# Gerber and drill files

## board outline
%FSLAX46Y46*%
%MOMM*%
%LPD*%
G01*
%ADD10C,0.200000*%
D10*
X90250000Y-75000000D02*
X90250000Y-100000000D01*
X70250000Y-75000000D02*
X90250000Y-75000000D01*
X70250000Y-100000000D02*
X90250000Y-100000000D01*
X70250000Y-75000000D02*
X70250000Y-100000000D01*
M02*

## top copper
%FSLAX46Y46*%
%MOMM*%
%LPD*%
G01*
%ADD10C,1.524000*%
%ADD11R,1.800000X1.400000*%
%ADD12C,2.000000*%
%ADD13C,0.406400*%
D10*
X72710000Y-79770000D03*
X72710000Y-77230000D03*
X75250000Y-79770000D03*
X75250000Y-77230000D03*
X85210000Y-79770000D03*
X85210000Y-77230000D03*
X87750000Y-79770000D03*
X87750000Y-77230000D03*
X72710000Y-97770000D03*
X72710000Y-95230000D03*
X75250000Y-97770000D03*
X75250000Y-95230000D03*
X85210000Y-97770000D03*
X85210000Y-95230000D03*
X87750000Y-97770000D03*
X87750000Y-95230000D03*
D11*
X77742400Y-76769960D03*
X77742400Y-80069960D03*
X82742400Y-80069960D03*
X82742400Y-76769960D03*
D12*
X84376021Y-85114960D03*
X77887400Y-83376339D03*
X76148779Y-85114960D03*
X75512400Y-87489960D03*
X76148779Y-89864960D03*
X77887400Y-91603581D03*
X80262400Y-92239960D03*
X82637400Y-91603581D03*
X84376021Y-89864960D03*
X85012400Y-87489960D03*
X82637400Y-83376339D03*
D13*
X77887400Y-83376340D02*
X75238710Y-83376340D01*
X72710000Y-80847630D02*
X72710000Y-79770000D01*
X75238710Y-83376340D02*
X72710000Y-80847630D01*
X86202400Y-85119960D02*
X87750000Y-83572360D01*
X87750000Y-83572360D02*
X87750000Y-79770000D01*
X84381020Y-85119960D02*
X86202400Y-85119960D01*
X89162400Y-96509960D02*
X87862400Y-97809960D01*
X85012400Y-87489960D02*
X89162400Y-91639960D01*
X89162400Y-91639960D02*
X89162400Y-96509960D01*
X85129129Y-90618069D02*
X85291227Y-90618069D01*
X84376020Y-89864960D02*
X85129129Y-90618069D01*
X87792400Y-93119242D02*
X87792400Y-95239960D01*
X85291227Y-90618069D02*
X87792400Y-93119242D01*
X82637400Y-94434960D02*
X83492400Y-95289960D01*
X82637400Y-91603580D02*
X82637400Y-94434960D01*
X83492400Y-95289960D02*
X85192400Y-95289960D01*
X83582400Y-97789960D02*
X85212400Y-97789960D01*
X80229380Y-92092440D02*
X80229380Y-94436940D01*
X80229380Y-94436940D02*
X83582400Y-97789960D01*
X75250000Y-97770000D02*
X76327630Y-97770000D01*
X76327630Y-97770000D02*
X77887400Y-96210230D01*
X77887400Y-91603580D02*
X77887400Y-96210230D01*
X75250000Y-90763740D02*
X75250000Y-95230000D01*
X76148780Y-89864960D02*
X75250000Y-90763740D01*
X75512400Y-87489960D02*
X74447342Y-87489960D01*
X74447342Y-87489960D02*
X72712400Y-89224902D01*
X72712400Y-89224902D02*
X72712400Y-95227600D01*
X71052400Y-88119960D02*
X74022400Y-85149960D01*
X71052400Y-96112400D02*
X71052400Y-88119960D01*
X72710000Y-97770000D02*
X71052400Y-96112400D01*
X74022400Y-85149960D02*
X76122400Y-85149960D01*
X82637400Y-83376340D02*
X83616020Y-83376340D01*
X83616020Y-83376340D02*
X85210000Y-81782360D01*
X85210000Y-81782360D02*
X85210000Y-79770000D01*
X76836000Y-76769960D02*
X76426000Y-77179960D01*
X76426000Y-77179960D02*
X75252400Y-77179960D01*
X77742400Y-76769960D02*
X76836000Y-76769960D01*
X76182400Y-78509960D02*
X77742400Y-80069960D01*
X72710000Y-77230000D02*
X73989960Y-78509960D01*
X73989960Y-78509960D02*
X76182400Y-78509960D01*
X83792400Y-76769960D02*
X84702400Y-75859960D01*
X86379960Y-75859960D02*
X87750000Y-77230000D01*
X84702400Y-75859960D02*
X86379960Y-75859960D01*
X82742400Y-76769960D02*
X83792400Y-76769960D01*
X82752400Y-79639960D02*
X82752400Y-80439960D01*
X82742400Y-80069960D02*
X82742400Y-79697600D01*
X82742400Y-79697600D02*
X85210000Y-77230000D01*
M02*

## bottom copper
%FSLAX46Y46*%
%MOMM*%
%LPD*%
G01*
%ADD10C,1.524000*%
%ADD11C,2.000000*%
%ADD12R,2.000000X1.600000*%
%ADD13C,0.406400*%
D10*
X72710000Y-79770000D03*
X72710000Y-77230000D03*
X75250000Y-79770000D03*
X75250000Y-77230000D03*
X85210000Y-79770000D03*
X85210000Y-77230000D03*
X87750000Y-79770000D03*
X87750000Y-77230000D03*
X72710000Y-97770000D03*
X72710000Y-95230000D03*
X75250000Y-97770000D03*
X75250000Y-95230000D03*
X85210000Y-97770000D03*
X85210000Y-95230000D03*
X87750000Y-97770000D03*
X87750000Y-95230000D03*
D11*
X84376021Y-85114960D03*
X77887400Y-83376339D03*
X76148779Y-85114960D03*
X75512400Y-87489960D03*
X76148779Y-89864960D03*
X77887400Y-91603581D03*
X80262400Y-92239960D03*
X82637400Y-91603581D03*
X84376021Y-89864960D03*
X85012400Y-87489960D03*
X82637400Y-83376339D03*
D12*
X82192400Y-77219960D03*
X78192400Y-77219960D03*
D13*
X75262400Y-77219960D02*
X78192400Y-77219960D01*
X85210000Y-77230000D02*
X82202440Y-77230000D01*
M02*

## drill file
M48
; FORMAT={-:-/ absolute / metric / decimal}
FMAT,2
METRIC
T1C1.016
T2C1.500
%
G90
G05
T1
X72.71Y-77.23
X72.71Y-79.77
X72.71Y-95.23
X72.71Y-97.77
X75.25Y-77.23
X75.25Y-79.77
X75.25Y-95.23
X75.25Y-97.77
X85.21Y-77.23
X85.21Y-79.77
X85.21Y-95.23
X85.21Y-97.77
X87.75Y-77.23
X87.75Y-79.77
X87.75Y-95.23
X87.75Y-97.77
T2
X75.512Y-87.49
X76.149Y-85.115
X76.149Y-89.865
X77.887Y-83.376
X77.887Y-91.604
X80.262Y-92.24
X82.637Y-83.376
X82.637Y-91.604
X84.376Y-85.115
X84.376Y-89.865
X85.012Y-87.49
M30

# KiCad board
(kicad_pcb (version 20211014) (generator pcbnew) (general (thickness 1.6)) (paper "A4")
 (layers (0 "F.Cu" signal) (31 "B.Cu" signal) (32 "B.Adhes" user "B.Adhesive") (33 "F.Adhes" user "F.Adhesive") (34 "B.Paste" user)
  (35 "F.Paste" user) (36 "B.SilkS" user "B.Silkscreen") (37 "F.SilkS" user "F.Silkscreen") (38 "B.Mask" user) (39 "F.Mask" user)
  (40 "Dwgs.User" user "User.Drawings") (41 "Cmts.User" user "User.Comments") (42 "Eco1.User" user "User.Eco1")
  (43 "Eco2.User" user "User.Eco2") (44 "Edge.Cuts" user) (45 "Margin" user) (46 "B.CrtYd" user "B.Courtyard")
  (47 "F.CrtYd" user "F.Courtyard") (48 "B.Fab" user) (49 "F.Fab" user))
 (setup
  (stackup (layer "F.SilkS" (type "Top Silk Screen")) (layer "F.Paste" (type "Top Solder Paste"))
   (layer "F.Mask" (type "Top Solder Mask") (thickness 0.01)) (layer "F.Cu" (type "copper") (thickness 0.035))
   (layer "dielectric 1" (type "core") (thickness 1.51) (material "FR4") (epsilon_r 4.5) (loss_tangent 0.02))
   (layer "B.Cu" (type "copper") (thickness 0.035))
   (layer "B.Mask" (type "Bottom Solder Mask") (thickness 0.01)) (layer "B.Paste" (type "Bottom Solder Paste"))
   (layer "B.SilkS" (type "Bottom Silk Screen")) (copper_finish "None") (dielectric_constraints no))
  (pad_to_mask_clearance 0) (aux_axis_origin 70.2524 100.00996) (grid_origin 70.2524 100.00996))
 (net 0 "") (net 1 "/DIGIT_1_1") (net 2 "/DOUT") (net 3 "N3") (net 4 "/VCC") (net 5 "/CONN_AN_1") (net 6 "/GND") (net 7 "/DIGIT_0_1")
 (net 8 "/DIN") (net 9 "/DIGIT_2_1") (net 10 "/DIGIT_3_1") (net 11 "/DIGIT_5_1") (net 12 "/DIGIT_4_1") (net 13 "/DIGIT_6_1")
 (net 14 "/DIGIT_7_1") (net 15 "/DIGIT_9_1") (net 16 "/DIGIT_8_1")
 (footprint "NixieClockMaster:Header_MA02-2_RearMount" (layer "F.Cu") (at 75.25 78.5)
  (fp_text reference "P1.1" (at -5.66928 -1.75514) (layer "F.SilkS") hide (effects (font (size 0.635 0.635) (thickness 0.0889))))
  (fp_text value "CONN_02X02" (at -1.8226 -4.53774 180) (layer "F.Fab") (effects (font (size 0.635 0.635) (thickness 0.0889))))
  (pad "1" thru_hole circle (at -2.54 1.27) (size 1.524 1.524) (drill 1.016) (layers *.Cu *.Mask) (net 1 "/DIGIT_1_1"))
  (pad "2" thru_hole circle (at -2.54 -1.27) (size 1.524 1.524) (drill 1.016) (layers *.Cu *.Mask) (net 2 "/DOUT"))
  (pad "3" thru_hole circle (at 0 1.27) (size 1.524 1.524) (drill 1.016) (layers *.Cu *.Mask) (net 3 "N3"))
  (pad "4" thru_hole circle (at 0 -1.27) (size 1.524 1.524) (drill 1.016) (layers *.Cu *.Mask) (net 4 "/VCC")))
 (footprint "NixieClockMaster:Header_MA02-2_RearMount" (layer "F.Cu") (at 87.75 78.5)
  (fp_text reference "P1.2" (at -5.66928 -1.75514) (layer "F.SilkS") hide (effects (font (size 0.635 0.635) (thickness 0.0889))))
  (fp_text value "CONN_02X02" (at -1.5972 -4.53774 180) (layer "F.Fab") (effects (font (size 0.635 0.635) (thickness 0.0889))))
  (pad "1" thru_hole circle (at -2.54 1.27) (size 1.524 1.524) (drill 1.016) (layers *.Cu *.Mask) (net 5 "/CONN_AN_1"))
  (pad "2" thru_hole circle (at -2.54 -1.27) (size 1.524 1.524) (drill 1.016) (layers *.Cu *.Mask) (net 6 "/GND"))
  (pad "3" thru_hole circle (at 0 1.27) (size 1.524 1.524) (drill 1.016) (layers *.Cu *.Mask) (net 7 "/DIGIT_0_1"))
  (pad "4" thru_hole circle (at 0 -1.27) (size 1.524 1.524) (drill 1.016) (layers *.Cu *.Mask) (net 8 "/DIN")))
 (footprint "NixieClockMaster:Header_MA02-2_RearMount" (layer "F.Cu") (at 75.25 96.5)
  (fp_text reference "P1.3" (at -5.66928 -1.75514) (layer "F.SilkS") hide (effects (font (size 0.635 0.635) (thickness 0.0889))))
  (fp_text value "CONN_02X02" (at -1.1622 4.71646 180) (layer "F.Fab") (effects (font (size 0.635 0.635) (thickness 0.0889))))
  (pad "1" thru_hole circle (at -2.54 1.27) (size 1.524 1.524) (drill 1.016) (layers *.Cu *.Mask) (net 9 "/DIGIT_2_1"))
  (pad "2" thru_hole circle (at -2.54 -1.27) (size 1.524 1.524) (drill 1.016) (layers *.Cu *.Mask) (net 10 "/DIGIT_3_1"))
  (pad "3" thru_hole circle (at 0 1.27) (size 1.524 1.524) (drill 1.016) (layers *.Cu *.Mask) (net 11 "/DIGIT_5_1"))
  (pad "4" thru_hole circle (at 0 -1.27) (size 1.524 1.524) (drill 1.016) (layers *.Cu *.Mask) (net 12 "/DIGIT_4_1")))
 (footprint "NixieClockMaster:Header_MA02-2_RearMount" (layer "F.Cu") (at 87.75 96.5)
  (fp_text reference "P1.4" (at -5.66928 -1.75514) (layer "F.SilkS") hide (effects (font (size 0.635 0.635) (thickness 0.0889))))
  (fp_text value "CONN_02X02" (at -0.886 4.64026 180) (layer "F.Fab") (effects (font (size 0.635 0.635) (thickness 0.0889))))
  (pad "1" thru_hole circle (at -2.54 1.27) (size 1.524 1.524) (drill 1.016) (layers *.Cu *.Mask) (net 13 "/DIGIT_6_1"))
  (pad "2" thru_hole circle (at -2.54 -1.27) (size 1.524 1.524) (drill 1.016) (layers *.Cu *.Mask) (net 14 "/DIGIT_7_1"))
  (pad "3" thru_hole circle (at 0 1.27) (size 1.524 1.524) (drill 1.016) (layers *.Cu *.Mask) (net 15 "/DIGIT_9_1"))
  (pad "4" thru_hole circle (at 0 -1.27) (size 1.524 1.524) (drill 1.016) (layers *.Cu *.Mask) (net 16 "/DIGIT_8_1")))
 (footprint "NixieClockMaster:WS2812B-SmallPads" (layer "F.Cu") (at 80.2424 78.41996 90)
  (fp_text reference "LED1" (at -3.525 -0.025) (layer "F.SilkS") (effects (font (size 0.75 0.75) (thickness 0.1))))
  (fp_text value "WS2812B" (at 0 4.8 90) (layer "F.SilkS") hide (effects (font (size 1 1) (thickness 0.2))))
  (pad "1" smd rect locked (at 1.65 -2.5 90) (size 1.4 1.8) (layers "F.Cu" "F.Paste" "F.Mask") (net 4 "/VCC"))
  (pad "2" smd rect locked (at -1.65 -2.5 90) (size 1.4 1.8) (layers "F.Cu" "F.Paste" "F.Mask") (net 2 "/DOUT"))
  (pad "3" smd rect locked (at -1.65 2.5 90) (size 1.4 1.8) (layers "F.Cu" "F.Paste" "F.Mask") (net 6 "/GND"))
  (pad "4" smd rect locked (at 1.65 2.5 90) (size 1.4 1.8) (layers "F.Cu" "F.Paste" "F.Mask") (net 8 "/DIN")))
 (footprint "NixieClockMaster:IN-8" (layer "F.Cu") (at 80.2624 87.48996)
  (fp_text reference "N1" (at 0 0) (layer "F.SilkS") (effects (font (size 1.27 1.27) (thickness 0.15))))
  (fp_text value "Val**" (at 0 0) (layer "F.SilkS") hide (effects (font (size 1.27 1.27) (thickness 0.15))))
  (pad "0" thru_hole circle locked (at 4.113621 -2.375 30) (size 2 2) (drill 1.5) (layers *.Cu *.Mask) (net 7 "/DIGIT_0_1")
   (solder_mask_margin 0.1016))
  (pad "1" thru_hole circle locked (at -2.375 -4.113621 120) (size 2 2) (drill 1.5) (layers *.Cu *.Mask) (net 1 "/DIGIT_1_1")
   (solder_mask_margin 0.1016))
  (pad "2" thru_hole circle locked (at -4.113621 -2.375 150) (size 2 2) (drill 1.5) (layers *.Cu *.Mask) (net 9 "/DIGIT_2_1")
   (solder_mask_margin 0.1016))
  (pad "3" thru_hole circle locked (at -4.75 0 180) (size 2 2) (drill 1.5) (layers *.Cu *.Mask) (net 10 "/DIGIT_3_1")
   (solder_mask_margin 0.1016))
  (pad "4" thru_hole circle locked (at -4.113621 2.375 210) (size 2 2) (drill 1.5) (layers *.Cu *.Mask) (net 12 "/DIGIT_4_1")
   (solder_mask_margin 0.1016))
  (pad "5" thru_hole circle locked (at -2.375 4.113621 240) (size 2 2) (drill 1.5) (layers *.Cu *.Mask) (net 11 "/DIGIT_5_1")
   (solder_mask_margin 0.1016))
  (pad "6" thru_hole circle locked (at 0 4.75 270) (size 2 2) (drill 1.5) (layers *.Cu *.Mask) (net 13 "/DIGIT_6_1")
   (solder_mask_margin 0.1016))
  (pad "7" thru_hole circle locked (at 2.375 4.113621 300) (size 2 2) (drill 1.5) (layers *.Cu *.Mask) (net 14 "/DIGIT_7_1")
   (solder_mask_margin 0.1016))
  (pad "8" thru_hole circle locked (at 4.113621 2.375 330) (size 2 2) (drill 1.5) (layers *.Cu *.Mask) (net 16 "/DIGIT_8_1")
   (solder_mask_margin 0.1016))
  (pad "9" thru_hole circle locked (at 4.75 0) (size 2 2) (drill 1.5) (layers *.Cu *.Mask) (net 15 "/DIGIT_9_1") (solder_mask_margin 0.1016))
  (pad "A" thru_hole circle locked (at 2.375 -4.113621 60) (size 2 2) (drill 1.5) (layers *.Cu *.Mask) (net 5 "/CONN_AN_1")
   (solder_mask_margin 0.1016)))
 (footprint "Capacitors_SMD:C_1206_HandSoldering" (layer "B.Cu") (at 80.1924 77.21996 180)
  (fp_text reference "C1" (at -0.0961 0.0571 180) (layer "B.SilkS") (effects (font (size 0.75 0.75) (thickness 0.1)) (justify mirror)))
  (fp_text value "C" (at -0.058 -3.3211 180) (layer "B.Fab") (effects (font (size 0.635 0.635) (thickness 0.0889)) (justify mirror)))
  (pad "1" smd rect locked (at -2 0 180) (size 2 1.6) (layers "B.Cu" "B.Paste" "B.Mask") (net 6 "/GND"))
  (pad "2" smd rect locked (at 2 0 180) (size 2 1.6) (layers "B.Cu" "B.Paste" "B.Mask") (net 4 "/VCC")))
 (gr_line (start 90.25 75) (end 90.25 100) (layer "Edge.Cuts") (width 0.2))
 (gr_line (start 70.25 75) (end 90.25 75) (layer "Edge.Cuts") (width 0.2))
 (gr_line (start 70.25 100) (end 90.25 100) (layer "Edge.Cuts") (width 0.2))
 (gr_line (start 70.25 75) (end 70.25 100) (layer "Edge.Cuts") (width 0.2))
 (segment (start 77.8874 83.37634) (end 75.23871 83.37634) (width 0.4064) (layer "F.Cu") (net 1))
 (segment (start 72.71 80.84763) (end 72.71 79.77) (width 0.4064) (layer "F.Cu") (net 1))
 (segment (start 75.23871 83.37634) (end 72.71 80.84763) (width 0.4064) (layer "F.Cu") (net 1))
 (segment (start 86.2024 85.11996) (end 87.75 83.57236) (width 0.4064) (layer "F.Cu") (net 7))
 (segment (start 87.75 83.57236) (end 87.75 79.77) (width 0.4064) (layer "F.Cu") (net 7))
 (segment (start 84.38102 85.11996) (end 86.2024 85.11996) (width 0.4064) (layer "F.Cu") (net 7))
 (segment (start 89.1624 96.50996) (end 87.8624 97.80996) (width 0.4064) (layer "F.Cu") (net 15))
 (segment (start 85.0124 87.48996) (end 89.1624 91.63996) (width 0.4064) (layer "F.Cu") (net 15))
 (segment (start 89.1624 91.63996) (end 89.1624 96.50996) (width 0.4064) (layer "F.Cu") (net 15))
 (segment (start 85.129129 90.618069) (end 85.291227 90.618069) (width 0.4064) (layer "F.Cu") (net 16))
 (segment (start 84.37602 89.86496) (end 85.129129 90.618069) (width 0.4064) (layer "F.Cu") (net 16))
 (segment (start 87.7924 93.119242) (end 87.7924 95.23996) (width 0.4064) (layer "F.Cu") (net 16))
 (segment (start 85.291227 90.618069) (end 87.7924 93.119242) (width 0.4064) (layer "F.Cu") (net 16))
 (segment (start 82.6374 94.43496) (end 83.4924 95.28996) (width 0.4064) (layer "F.Cu") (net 14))
 (segment (start 82.6374 91.60358) (end 82.6374 94.43496) (width 0.4064) (layer "F.Cu") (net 14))
 (segment (start 83.4924 95.28996) (end 85.1924 95.28996) (width 0.4064) (layer "F.Cu") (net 14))
 (segment (start 83.5824 97.78996) (end 85.2124 97.78996) (width 0.4064) (layer "F.Cu") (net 13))
 (segment (start 80.22938 92.09244) (end 80.22938 94.43694) (width 0.4064) (layer "F.Cu") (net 13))
 (segment (start 80.22938 94.43694) (end 83.5824 97.78996) (width 0.4064) (layer "F.Cu") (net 13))
 (segment (start 75.25 97.77) (end 76.32763 97.77) (width 0.4064) (layer "F.Cu") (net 11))
 (segment (start 76.32763 97.77) (end 77.8874 96.21023) (width 0.4064) (layer "F.Cu") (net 11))
 (segment (start 77.8874 91.60358) (end 77.8874 96.21023) (width 0.4064) (layer "F.Cu") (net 11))
 (segment (start 75.25 90.76374) (end 75.25 95.23) (width 0.4064) (layer "F.Cu") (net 12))
 (segment (start 76.14878 89.86496) (end 75.25 90.76374) (width 0.4064) (layer "F.Cu") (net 12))
 (segment (start 75.5124 87.48996) (end 74.447342 87.48996) (width 0.4064) (layer "F.Cu") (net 10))
 (segment (start 74.447342 87.48996) (end 72.7124 89.224902) (width 0.4064) (layer "F.Cu") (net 10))
 (segment (start 72.7124 89.224902) (end 72.7124 95.2276) (width 0.4064) (layer "F.Cu") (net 10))
 (segment (start 71.0524 88.11996) (end 74.0224 85.14996) (width 0.4064) (layer "F.Cu") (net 9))
 (segment (start 71.0524 96.1124) (end 71.0524 88.11996) (width 0.4064) (layer "F.Cu") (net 9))
 (segment (start 72.71 97.77) (end 71.0524 96.1124) (width 0.4064) (layer "F.Cu") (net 9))
 (segment (start 74.0224 85.14996) (end 76.1224 85.14996) (width 0.4064) (layer "F.Cu") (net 9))
 (segment (start 82.6374 83.37634) (end 83.61602 83.37634) (width 0.4064) (layer "F.Cu") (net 5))
 (segment (start 83.61602 83.37634) (end 85.21 81.78236) (width 0.4064) (layer "F.Cu") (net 5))
 (segment (start 85.21 81.78236) (end 85.21 79.77) (width 0.4064) (layer "F.Cu") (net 5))
 (segment (start 76.836 76.76996) (end 76.426 77.17996) (width 0.4064) (layer "F.Cu") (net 4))
 (segment (start 76.426 77.17996) (end 75.2524 77.17996) (width 0.4064) (layer "F.Cu") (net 4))
 (segment (start 77.7424 76.76996) (end 76.836 76.76996) (width 0.4064) (layer "F.Cu") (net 4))
 (segment (start 75.2624 77.21996) (end 78.1924 77.21996) (width 0.4064) (layer "B.Cu") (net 4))
 (segment (start 76.1824 78.50996) (end 77.7424 80.06996) (width 0.4064) (layer "F.Cu") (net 2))
 (segment (start 72.71 77.23) (end 73.98996 78.50996) (width 0.4064) (layer "F.Cu") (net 2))
 (segment (start 73.98996 78.50996) (end 76.1824 78.50996) (width 0.4064) (layer "F.Cu") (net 2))
 (segment (start 83.7924 76.76996) (end 84.7024 75.85996) (width 0.4064) (layer "F.Cu") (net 8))
 (segment (start 86.37996 75.85996) (end 87.75 77.23) (width 0.4064) (layer "F.Cu") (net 8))
 (segment (start 84.7024 75.85996) (end 86.37996 75.85996) (width 0.4064) (layer "F.Cu") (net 8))
 (segment (start 82.7424 76.76996) (end 83.7924 76.76996) (width 0.4064) (layer "F.Cu") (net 8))
 (segment (start 82.7524 79.63996) (end 82.7524 80.43996) (width 0.4064) (layer "F.Cu") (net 6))
 (segment (start 82.7424 80.06996) (end 82.7424 79.6976) (width 0.4064) (layer "F.Cu") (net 6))
 (segment (start 82.7424 79.6976) (end 85.21 77.23) (width 0.4064) (layer "F.Cu") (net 6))
 (segment (start 85.21 77.23) (end 82.20244 77.23) (width 0.4064) (layer "B.Cu") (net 6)))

